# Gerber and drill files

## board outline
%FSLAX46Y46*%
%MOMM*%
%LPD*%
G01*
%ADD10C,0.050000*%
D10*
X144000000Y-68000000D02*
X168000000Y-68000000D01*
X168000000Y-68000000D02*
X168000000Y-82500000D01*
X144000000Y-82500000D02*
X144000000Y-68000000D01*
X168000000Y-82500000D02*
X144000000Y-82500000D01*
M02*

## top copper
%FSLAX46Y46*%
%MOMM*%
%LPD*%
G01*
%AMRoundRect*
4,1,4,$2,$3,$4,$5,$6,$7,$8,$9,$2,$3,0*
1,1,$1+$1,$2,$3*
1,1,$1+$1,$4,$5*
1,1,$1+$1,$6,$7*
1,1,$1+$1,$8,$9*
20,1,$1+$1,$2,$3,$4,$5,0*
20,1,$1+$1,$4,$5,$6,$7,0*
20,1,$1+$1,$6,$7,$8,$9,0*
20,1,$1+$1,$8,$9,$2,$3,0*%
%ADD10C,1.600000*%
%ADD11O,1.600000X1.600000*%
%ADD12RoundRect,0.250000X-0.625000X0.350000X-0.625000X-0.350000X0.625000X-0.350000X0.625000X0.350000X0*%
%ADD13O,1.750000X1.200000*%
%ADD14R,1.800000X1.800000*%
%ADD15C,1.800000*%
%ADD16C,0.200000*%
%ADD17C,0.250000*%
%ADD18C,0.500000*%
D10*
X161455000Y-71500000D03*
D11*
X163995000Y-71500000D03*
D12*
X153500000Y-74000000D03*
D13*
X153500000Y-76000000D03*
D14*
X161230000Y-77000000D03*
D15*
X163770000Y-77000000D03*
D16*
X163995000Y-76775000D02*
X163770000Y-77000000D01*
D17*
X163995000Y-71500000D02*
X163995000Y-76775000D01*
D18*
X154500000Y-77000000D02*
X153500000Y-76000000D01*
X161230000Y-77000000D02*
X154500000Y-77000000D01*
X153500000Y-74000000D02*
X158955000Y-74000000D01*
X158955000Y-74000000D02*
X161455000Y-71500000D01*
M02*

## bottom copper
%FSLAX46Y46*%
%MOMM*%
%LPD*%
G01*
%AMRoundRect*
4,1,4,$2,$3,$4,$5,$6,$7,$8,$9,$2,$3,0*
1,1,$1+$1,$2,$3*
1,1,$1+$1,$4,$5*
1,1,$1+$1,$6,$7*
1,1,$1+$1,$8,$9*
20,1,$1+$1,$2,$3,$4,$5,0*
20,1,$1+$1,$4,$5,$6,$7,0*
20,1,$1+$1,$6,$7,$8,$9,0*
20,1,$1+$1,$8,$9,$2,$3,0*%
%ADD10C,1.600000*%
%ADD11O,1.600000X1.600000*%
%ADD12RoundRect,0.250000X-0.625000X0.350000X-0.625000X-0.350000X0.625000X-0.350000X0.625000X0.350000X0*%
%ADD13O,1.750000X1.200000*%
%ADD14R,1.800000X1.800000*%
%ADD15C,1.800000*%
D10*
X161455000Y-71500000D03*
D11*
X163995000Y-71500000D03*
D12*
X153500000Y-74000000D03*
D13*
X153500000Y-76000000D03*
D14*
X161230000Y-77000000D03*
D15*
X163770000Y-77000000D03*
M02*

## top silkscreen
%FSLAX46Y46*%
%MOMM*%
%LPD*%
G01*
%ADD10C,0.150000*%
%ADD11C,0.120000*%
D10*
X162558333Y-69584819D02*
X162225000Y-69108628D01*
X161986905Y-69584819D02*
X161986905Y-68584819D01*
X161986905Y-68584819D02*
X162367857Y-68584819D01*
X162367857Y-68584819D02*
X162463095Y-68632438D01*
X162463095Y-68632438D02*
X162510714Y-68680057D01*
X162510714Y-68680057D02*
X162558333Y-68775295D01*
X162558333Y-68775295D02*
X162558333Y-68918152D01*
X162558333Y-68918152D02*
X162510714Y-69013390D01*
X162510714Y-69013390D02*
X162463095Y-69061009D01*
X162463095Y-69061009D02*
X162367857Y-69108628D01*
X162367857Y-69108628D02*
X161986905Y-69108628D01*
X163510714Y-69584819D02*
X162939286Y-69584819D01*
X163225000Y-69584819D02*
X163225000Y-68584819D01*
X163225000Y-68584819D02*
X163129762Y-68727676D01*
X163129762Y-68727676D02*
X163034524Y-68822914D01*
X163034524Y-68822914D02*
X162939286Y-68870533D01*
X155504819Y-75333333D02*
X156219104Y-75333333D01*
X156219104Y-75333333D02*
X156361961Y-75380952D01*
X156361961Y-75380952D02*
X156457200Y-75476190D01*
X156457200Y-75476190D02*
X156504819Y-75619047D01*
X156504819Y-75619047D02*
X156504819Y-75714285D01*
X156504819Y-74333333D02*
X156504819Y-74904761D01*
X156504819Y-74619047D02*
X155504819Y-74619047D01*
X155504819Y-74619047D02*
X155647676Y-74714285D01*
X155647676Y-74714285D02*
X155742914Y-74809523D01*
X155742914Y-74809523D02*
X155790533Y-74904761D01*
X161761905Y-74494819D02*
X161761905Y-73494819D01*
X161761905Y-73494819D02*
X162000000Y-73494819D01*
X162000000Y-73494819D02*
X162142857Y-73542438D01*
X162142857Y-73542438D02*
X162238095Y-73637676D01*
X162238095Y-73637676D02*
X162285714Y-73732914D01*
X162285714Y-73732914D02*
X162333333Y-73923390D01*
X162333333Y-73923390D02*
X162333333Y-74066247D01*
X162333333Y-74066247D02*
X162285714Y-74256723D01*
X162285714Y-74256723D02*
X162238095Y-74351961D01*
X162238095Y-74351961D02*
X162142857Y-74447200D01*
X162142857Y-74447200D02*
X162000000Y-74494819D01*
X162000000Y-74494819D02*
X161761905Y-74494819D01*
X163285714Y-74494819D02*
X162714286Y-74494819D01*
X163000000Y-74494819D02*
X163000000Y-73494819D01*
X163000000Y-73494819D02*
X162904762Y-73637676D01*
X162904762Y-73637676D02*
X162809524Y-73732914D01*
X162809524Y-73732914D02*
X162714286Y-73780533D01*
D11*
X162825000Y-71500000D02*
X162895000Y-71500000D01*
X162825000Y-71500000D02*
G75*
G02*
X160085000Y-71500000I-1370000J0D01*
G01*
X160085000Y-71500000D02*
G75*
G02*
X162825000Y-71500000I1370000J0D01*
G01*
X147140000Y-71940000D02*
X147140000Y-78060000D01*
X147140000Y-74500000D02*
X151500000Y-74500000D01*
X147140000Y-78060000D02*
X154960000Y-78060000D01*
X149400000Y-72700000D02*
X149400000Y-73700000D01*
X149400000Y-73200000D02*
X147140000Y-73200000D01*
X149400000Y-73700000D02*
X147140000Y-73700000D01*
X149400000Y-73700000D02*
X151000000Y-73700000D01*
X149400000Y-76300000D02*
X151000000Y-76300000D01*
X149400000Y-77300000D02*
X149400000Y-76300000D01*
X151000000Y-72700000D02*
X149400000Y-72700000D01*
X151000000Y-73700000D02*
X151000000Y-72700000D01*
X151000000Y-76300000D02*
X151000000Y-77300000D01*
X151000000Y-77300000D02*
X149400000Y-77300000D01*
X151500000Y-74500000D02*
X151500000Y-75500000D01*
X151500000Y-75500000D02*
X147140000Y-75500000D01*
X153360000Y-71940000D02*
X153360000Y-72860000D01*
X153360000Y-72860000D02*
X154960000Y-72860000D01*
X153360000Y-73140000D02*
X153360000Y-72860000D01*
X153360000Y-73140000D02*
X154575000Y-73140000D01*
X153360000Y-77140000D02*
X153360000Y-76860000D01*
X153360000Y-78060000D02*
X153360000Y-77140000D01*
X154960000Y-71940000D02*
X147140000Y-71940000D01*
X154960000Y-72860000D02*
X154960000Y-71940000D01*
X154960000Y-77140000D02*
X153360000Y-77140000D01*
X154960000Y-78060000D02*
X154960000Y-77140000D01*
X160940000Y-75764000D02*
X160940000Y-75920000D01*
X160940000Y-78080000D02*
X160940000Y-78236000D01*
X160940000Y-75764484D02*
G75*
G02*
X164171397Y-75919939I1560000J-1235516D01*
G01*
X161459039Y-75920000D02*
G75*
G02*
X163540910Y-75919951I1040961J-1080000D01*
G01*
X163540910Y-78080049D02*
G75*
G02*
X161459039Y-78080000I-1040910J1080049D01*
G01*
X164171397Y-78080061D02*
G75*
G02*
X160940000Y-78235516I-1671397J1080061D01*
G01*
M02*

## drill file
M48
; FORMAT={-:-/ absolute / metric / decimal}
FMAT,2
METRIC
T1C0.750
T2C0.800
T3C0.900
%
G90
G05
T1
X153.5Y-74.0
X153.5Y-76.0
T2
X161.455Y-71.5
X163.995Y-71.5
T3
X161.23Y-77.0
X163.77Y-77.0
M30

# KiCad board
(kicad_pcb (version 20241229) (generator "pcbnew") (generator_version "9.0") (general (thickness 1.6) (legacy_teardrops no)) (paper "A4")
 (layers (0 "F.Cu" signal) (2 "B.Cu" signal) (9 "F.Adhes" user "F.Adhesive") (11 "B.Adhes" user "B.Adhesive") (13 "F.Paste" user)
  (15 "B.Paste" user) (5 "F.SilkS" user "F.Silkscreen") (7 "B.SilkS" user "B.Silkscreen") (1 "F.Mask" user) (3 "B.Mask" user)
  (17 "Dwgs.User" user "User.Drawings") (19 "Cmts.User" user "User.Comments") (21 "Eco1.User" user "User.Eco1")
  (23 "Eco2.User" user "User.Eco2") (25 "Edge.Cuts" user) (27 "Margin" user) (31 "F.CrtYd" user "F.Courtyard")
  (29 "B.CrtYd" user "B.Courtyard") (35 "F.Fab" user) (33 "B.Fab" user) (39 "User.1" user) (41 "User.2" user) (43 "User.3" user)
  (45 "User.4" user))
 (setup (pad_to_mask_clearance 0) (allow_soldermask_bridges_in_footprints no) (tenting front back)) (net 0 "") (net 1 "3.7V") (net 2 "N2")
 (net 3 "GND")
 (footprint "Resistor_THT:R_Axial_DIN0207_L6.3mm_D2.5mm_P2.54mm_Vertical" (layer "F.Cu") (at 161.455 71.5)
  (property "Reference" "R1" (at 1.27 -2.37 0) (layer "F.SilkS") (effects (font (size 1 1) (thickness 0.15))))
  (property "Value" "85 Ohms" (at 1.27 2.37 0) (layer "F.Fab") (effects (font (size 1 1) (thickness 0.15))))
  (fp_line (start 1.37 0) (end 1.44 0) (stroke (width 0.12) (type solid)) (layer "F.SilkS"))
  (fp_circle (center 0 0) (end 1.37 0) (stroke (width 0.12) (type solid)) (fill no) (layer "F.SilkS"))
  (pad "1" thru_hole circle (at 0 0) (size 1.6 1.6) (drill 0.8) (layers "*.Cu" "*.Mask") (remove_unused_layers no) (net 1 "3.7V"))
  (pad "2" thru_hole oval (at 2.54 0) (size 1.6 1.6) (drill 0.8) (layers "*.Cu" "*.Mask") (remove_unused_layers no) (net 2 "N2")))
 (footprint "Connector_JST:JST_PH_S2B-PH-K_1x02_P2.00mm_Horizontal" (layer "F.Cu") (at 153.5 74 -90)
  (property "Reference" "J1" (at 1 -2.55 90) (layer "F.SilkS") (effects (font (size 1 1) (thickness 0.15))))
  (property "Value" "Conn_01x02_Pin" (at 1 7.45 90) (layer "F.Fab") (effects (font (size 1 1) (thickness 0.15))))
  (fp_line (start -2.06 6.36) (end 4.06 6.36) (stroke (width 0.12) (type solid)) (layer "F.SilkS"))
  (fp_line (start 0.5 6.36) (end 0.5 2) (stroke (width 0.12) (type solid)) (layer "F.SilkS"))
  (fp_line (start 4.06 6.36) (end 4.06 -1.46) (stroke (width 0.12) (type solid)) (layer "F.SilkS"))
  (fp_line (start -1.3 4.1) (end -0.3 4.1) (stroke (width 0.12) (type solid)) (layer "F.SilkS"))
  (fp_line (start -0.8 4.1) (end -0.8 6.36) (stroke (width 0.12) (type solid)) (layer "F.SilkS"))
  (fp_line (start -0.3 4.1) (end -0.3 6.36) (stroke (width 0.12) (type solid)) (layer "F.SilkS"))
  (fp_line (start -0.3 4.1) (end -0.3 2.5) (stroke (width 0.12) (type solid)) (layer "F.SilkS"))
  (fp_line (start 2.3 4.1) (end 2.3 2.5) (stroke (width 0.12) (type solid)) (layer "F.SilkS"))
  (fp_line (start 3.3 4.1) (end 2.3 4.1) (stroke (width 0.12) (type solid)) (layer "F.SilkS"))
  (fp_line (start -1.3 2.5) (end -1.3 4.1) (stroke (width 0.12) (type solid)) (layer "F.SilkS"))
  (fp_line (start -0.3 2.5) (end -1.3 2.5) (stroke (width 0.12) (type solid)) (layer "F.SilkS"))
  (fp_line (start 2.3 2.5) (end 3.3 2.5) (stroke (width 0.12) (type solid)) (layer "F.SilkS"))
  (fp_line (start 3.3 2.5) (end 3.3 4.1) (stroke (width 0.12) (type solid)) (layer "F.SilkS"))
  (fp_line (start 0.5 2) (end 1.5 2) (stroke (width 0.12) (type solid)) (layer "F.SilkS"))
  (fp_line (start 1.5 2) (end 1.5 6.36) (stroke (width 0.12) (type solid)) (layer "F.SilkS"))
  (fp_line (start -2.06 0.14) (end -1.14 0.14) (stroke (width 0.12) (type solid)) (layer "F.SilkS"))
  (fp_line (start -1.14 0.14) (end -1.14 -1.46) (stroke (width 0.12) (type solid)) (layer "F.SilkS"))
  (fp_line (start -0.86 0.14) (end -1.14 0.14) (stroke (width 0.12) (type solid)) (layer "F.SilkS"))
  (fp_line (start -0.86 0.14) (end -0.86 -1.075) (stroke (width 0.12) (type solid)) (layer "F.SilkS"))
  (fp_line (start 3.14 0.14) (end 2.86 0.14) (stroke (width 0.12) (type solid)) (layer "F.SilkS"))
  (fp_line (start 4.06 0.14) (end 3.14 0.14) (stroke (width 0.12) (type solid)) (layer "F.SilkS"))
  (fp_line (start -2.06 -1.46) (end -2.06 6.36) (stroke (width 0.12) (type solid)) (layer "F.SilkS"))
  (fp_line (start -1.14 -1.46) (end -2.06 -1.46) (stroke (width 0.12) (type solid)) (layer "F.SilkS"))
  (fp_line (start 3.14 -1.46) (end 3.14 0.14) (stroke (width 0.12) (type solid)) (layer "F.SilkS"))
  (fp_line (start 4.06 -1.46) (end 3.14 -1.46) (stroke (width 0.12) (type solid)) (layer "F.SilkS"))
  (pad "1" thru_hole roundrect (at 0 0 270) (size 1.2 1.75) (drill 0.75) (layers "*.Cu" "*.Mask") (remove_unused_layers no)
   (roundrect_rratio 0.208333) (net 1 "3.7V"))
  (pad "2" thru_hole oval (at 2 0 270) (size 1.2 1.75) (drill 0.75) (layers "*.Cu" "*.Mask") (remove_unused_layers no) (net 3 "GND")))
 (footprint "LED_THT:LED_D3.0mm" (layer "F.Cu") (at 161.23 77)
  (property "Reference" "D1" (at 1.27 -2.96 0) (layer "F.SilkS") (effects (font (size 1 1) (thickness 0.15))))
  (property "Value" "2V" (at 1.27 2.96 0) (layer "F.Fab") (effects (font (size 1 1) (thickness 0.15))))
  (fp_line (start -0.29 -1.236) (end -0.29 -1.08) (stroke (width 0.12) (type solid)) (layer "F.SilkS"))
  (fp_line (start -0.29 1.08) (end -0.29 1.236) (stroke (width 0.12) (type solid)) (layer "F.SilkS"))
  (fp_arc (start -0.29 -1.235516) (mid 1.365624 -1.987701) (end 2.941397 -1.080061) (stroke (width 0.12) (type solid)) (layer "F.SilkS"))
  (fp_arc (start 0.229039 -1.08) (mid 1.269964 -1.5) (end 2.31091 -1.080049) (stroke (width 0.12) (type solid)) (layer "F.SilkS"))
  (fp_arc (start 2.31091 1.080049) (mid 1.269964 1.5) (end 0.229039 1.08) (stroke (width 0.12) (type solid)) (layer "F.SilkS"))
  (fp_arc (start 2.941397 1.080061) (mid 1.365624 1.987701) (end -0.29 1.235516) (stroke (width 0.12) (type solid)) (layer "F.SilkS"))
  (pad "1" thru_hole rect (at 0 0) (size 1.8 1.8) (drill 0.9) (layers "*.Cu" "*.Mask") (remove_unused_layers no) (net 3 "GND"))
  (pad "2" thru_hole circle (at 2.54 0) (size 1.8 1.8) (drill 0.9) (layers "*.Cu" "*.Mask") (remove_unused_layers no) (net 2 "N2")))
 (gr_line (start 144 68) (end 168 68) (stroke (width 0.05) (type default)) (layer "Edge.Cuts"))
 (gr_line (start 168 68) (end 168 82.5) (stroke (width 0.05) (type default)) (layer "Edge.Cuts"))
 (gr_line (start 144 82.5) (end 144 68) (stroke (width 0.05) (type default)) (layer "Edge.Cuts"))
 (gr_line (start 168 82.5) (end 144 82.5) (stroke (width 0.05) (type default)) (layer "Edge.Cuts"))
 (segment (start 163.995 76.775) (end 163.77 77) (width 0.2) (layer "F.Cu") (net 2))
 (segment (start 163.995 71.5) (end 163.995 76.775) (width 0.25) (layer "F.Cu") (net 2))
 (segment (start 154.5 77) (end 153.5 76) (width 0.5) (layer "F.Cu") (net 3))
 (segment (start 161.23 77) (end 154.5 77) (width 0.5) (layer "F.Cu") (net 3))
 (segment (start 153.5 74) (end 158.955 74) (width 0.5) (layer "F.Cu") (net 1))
 (segment (start 158.955 74) (end 161.455 71.5) (width 0.5) (layer "F.Cu") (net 1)))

